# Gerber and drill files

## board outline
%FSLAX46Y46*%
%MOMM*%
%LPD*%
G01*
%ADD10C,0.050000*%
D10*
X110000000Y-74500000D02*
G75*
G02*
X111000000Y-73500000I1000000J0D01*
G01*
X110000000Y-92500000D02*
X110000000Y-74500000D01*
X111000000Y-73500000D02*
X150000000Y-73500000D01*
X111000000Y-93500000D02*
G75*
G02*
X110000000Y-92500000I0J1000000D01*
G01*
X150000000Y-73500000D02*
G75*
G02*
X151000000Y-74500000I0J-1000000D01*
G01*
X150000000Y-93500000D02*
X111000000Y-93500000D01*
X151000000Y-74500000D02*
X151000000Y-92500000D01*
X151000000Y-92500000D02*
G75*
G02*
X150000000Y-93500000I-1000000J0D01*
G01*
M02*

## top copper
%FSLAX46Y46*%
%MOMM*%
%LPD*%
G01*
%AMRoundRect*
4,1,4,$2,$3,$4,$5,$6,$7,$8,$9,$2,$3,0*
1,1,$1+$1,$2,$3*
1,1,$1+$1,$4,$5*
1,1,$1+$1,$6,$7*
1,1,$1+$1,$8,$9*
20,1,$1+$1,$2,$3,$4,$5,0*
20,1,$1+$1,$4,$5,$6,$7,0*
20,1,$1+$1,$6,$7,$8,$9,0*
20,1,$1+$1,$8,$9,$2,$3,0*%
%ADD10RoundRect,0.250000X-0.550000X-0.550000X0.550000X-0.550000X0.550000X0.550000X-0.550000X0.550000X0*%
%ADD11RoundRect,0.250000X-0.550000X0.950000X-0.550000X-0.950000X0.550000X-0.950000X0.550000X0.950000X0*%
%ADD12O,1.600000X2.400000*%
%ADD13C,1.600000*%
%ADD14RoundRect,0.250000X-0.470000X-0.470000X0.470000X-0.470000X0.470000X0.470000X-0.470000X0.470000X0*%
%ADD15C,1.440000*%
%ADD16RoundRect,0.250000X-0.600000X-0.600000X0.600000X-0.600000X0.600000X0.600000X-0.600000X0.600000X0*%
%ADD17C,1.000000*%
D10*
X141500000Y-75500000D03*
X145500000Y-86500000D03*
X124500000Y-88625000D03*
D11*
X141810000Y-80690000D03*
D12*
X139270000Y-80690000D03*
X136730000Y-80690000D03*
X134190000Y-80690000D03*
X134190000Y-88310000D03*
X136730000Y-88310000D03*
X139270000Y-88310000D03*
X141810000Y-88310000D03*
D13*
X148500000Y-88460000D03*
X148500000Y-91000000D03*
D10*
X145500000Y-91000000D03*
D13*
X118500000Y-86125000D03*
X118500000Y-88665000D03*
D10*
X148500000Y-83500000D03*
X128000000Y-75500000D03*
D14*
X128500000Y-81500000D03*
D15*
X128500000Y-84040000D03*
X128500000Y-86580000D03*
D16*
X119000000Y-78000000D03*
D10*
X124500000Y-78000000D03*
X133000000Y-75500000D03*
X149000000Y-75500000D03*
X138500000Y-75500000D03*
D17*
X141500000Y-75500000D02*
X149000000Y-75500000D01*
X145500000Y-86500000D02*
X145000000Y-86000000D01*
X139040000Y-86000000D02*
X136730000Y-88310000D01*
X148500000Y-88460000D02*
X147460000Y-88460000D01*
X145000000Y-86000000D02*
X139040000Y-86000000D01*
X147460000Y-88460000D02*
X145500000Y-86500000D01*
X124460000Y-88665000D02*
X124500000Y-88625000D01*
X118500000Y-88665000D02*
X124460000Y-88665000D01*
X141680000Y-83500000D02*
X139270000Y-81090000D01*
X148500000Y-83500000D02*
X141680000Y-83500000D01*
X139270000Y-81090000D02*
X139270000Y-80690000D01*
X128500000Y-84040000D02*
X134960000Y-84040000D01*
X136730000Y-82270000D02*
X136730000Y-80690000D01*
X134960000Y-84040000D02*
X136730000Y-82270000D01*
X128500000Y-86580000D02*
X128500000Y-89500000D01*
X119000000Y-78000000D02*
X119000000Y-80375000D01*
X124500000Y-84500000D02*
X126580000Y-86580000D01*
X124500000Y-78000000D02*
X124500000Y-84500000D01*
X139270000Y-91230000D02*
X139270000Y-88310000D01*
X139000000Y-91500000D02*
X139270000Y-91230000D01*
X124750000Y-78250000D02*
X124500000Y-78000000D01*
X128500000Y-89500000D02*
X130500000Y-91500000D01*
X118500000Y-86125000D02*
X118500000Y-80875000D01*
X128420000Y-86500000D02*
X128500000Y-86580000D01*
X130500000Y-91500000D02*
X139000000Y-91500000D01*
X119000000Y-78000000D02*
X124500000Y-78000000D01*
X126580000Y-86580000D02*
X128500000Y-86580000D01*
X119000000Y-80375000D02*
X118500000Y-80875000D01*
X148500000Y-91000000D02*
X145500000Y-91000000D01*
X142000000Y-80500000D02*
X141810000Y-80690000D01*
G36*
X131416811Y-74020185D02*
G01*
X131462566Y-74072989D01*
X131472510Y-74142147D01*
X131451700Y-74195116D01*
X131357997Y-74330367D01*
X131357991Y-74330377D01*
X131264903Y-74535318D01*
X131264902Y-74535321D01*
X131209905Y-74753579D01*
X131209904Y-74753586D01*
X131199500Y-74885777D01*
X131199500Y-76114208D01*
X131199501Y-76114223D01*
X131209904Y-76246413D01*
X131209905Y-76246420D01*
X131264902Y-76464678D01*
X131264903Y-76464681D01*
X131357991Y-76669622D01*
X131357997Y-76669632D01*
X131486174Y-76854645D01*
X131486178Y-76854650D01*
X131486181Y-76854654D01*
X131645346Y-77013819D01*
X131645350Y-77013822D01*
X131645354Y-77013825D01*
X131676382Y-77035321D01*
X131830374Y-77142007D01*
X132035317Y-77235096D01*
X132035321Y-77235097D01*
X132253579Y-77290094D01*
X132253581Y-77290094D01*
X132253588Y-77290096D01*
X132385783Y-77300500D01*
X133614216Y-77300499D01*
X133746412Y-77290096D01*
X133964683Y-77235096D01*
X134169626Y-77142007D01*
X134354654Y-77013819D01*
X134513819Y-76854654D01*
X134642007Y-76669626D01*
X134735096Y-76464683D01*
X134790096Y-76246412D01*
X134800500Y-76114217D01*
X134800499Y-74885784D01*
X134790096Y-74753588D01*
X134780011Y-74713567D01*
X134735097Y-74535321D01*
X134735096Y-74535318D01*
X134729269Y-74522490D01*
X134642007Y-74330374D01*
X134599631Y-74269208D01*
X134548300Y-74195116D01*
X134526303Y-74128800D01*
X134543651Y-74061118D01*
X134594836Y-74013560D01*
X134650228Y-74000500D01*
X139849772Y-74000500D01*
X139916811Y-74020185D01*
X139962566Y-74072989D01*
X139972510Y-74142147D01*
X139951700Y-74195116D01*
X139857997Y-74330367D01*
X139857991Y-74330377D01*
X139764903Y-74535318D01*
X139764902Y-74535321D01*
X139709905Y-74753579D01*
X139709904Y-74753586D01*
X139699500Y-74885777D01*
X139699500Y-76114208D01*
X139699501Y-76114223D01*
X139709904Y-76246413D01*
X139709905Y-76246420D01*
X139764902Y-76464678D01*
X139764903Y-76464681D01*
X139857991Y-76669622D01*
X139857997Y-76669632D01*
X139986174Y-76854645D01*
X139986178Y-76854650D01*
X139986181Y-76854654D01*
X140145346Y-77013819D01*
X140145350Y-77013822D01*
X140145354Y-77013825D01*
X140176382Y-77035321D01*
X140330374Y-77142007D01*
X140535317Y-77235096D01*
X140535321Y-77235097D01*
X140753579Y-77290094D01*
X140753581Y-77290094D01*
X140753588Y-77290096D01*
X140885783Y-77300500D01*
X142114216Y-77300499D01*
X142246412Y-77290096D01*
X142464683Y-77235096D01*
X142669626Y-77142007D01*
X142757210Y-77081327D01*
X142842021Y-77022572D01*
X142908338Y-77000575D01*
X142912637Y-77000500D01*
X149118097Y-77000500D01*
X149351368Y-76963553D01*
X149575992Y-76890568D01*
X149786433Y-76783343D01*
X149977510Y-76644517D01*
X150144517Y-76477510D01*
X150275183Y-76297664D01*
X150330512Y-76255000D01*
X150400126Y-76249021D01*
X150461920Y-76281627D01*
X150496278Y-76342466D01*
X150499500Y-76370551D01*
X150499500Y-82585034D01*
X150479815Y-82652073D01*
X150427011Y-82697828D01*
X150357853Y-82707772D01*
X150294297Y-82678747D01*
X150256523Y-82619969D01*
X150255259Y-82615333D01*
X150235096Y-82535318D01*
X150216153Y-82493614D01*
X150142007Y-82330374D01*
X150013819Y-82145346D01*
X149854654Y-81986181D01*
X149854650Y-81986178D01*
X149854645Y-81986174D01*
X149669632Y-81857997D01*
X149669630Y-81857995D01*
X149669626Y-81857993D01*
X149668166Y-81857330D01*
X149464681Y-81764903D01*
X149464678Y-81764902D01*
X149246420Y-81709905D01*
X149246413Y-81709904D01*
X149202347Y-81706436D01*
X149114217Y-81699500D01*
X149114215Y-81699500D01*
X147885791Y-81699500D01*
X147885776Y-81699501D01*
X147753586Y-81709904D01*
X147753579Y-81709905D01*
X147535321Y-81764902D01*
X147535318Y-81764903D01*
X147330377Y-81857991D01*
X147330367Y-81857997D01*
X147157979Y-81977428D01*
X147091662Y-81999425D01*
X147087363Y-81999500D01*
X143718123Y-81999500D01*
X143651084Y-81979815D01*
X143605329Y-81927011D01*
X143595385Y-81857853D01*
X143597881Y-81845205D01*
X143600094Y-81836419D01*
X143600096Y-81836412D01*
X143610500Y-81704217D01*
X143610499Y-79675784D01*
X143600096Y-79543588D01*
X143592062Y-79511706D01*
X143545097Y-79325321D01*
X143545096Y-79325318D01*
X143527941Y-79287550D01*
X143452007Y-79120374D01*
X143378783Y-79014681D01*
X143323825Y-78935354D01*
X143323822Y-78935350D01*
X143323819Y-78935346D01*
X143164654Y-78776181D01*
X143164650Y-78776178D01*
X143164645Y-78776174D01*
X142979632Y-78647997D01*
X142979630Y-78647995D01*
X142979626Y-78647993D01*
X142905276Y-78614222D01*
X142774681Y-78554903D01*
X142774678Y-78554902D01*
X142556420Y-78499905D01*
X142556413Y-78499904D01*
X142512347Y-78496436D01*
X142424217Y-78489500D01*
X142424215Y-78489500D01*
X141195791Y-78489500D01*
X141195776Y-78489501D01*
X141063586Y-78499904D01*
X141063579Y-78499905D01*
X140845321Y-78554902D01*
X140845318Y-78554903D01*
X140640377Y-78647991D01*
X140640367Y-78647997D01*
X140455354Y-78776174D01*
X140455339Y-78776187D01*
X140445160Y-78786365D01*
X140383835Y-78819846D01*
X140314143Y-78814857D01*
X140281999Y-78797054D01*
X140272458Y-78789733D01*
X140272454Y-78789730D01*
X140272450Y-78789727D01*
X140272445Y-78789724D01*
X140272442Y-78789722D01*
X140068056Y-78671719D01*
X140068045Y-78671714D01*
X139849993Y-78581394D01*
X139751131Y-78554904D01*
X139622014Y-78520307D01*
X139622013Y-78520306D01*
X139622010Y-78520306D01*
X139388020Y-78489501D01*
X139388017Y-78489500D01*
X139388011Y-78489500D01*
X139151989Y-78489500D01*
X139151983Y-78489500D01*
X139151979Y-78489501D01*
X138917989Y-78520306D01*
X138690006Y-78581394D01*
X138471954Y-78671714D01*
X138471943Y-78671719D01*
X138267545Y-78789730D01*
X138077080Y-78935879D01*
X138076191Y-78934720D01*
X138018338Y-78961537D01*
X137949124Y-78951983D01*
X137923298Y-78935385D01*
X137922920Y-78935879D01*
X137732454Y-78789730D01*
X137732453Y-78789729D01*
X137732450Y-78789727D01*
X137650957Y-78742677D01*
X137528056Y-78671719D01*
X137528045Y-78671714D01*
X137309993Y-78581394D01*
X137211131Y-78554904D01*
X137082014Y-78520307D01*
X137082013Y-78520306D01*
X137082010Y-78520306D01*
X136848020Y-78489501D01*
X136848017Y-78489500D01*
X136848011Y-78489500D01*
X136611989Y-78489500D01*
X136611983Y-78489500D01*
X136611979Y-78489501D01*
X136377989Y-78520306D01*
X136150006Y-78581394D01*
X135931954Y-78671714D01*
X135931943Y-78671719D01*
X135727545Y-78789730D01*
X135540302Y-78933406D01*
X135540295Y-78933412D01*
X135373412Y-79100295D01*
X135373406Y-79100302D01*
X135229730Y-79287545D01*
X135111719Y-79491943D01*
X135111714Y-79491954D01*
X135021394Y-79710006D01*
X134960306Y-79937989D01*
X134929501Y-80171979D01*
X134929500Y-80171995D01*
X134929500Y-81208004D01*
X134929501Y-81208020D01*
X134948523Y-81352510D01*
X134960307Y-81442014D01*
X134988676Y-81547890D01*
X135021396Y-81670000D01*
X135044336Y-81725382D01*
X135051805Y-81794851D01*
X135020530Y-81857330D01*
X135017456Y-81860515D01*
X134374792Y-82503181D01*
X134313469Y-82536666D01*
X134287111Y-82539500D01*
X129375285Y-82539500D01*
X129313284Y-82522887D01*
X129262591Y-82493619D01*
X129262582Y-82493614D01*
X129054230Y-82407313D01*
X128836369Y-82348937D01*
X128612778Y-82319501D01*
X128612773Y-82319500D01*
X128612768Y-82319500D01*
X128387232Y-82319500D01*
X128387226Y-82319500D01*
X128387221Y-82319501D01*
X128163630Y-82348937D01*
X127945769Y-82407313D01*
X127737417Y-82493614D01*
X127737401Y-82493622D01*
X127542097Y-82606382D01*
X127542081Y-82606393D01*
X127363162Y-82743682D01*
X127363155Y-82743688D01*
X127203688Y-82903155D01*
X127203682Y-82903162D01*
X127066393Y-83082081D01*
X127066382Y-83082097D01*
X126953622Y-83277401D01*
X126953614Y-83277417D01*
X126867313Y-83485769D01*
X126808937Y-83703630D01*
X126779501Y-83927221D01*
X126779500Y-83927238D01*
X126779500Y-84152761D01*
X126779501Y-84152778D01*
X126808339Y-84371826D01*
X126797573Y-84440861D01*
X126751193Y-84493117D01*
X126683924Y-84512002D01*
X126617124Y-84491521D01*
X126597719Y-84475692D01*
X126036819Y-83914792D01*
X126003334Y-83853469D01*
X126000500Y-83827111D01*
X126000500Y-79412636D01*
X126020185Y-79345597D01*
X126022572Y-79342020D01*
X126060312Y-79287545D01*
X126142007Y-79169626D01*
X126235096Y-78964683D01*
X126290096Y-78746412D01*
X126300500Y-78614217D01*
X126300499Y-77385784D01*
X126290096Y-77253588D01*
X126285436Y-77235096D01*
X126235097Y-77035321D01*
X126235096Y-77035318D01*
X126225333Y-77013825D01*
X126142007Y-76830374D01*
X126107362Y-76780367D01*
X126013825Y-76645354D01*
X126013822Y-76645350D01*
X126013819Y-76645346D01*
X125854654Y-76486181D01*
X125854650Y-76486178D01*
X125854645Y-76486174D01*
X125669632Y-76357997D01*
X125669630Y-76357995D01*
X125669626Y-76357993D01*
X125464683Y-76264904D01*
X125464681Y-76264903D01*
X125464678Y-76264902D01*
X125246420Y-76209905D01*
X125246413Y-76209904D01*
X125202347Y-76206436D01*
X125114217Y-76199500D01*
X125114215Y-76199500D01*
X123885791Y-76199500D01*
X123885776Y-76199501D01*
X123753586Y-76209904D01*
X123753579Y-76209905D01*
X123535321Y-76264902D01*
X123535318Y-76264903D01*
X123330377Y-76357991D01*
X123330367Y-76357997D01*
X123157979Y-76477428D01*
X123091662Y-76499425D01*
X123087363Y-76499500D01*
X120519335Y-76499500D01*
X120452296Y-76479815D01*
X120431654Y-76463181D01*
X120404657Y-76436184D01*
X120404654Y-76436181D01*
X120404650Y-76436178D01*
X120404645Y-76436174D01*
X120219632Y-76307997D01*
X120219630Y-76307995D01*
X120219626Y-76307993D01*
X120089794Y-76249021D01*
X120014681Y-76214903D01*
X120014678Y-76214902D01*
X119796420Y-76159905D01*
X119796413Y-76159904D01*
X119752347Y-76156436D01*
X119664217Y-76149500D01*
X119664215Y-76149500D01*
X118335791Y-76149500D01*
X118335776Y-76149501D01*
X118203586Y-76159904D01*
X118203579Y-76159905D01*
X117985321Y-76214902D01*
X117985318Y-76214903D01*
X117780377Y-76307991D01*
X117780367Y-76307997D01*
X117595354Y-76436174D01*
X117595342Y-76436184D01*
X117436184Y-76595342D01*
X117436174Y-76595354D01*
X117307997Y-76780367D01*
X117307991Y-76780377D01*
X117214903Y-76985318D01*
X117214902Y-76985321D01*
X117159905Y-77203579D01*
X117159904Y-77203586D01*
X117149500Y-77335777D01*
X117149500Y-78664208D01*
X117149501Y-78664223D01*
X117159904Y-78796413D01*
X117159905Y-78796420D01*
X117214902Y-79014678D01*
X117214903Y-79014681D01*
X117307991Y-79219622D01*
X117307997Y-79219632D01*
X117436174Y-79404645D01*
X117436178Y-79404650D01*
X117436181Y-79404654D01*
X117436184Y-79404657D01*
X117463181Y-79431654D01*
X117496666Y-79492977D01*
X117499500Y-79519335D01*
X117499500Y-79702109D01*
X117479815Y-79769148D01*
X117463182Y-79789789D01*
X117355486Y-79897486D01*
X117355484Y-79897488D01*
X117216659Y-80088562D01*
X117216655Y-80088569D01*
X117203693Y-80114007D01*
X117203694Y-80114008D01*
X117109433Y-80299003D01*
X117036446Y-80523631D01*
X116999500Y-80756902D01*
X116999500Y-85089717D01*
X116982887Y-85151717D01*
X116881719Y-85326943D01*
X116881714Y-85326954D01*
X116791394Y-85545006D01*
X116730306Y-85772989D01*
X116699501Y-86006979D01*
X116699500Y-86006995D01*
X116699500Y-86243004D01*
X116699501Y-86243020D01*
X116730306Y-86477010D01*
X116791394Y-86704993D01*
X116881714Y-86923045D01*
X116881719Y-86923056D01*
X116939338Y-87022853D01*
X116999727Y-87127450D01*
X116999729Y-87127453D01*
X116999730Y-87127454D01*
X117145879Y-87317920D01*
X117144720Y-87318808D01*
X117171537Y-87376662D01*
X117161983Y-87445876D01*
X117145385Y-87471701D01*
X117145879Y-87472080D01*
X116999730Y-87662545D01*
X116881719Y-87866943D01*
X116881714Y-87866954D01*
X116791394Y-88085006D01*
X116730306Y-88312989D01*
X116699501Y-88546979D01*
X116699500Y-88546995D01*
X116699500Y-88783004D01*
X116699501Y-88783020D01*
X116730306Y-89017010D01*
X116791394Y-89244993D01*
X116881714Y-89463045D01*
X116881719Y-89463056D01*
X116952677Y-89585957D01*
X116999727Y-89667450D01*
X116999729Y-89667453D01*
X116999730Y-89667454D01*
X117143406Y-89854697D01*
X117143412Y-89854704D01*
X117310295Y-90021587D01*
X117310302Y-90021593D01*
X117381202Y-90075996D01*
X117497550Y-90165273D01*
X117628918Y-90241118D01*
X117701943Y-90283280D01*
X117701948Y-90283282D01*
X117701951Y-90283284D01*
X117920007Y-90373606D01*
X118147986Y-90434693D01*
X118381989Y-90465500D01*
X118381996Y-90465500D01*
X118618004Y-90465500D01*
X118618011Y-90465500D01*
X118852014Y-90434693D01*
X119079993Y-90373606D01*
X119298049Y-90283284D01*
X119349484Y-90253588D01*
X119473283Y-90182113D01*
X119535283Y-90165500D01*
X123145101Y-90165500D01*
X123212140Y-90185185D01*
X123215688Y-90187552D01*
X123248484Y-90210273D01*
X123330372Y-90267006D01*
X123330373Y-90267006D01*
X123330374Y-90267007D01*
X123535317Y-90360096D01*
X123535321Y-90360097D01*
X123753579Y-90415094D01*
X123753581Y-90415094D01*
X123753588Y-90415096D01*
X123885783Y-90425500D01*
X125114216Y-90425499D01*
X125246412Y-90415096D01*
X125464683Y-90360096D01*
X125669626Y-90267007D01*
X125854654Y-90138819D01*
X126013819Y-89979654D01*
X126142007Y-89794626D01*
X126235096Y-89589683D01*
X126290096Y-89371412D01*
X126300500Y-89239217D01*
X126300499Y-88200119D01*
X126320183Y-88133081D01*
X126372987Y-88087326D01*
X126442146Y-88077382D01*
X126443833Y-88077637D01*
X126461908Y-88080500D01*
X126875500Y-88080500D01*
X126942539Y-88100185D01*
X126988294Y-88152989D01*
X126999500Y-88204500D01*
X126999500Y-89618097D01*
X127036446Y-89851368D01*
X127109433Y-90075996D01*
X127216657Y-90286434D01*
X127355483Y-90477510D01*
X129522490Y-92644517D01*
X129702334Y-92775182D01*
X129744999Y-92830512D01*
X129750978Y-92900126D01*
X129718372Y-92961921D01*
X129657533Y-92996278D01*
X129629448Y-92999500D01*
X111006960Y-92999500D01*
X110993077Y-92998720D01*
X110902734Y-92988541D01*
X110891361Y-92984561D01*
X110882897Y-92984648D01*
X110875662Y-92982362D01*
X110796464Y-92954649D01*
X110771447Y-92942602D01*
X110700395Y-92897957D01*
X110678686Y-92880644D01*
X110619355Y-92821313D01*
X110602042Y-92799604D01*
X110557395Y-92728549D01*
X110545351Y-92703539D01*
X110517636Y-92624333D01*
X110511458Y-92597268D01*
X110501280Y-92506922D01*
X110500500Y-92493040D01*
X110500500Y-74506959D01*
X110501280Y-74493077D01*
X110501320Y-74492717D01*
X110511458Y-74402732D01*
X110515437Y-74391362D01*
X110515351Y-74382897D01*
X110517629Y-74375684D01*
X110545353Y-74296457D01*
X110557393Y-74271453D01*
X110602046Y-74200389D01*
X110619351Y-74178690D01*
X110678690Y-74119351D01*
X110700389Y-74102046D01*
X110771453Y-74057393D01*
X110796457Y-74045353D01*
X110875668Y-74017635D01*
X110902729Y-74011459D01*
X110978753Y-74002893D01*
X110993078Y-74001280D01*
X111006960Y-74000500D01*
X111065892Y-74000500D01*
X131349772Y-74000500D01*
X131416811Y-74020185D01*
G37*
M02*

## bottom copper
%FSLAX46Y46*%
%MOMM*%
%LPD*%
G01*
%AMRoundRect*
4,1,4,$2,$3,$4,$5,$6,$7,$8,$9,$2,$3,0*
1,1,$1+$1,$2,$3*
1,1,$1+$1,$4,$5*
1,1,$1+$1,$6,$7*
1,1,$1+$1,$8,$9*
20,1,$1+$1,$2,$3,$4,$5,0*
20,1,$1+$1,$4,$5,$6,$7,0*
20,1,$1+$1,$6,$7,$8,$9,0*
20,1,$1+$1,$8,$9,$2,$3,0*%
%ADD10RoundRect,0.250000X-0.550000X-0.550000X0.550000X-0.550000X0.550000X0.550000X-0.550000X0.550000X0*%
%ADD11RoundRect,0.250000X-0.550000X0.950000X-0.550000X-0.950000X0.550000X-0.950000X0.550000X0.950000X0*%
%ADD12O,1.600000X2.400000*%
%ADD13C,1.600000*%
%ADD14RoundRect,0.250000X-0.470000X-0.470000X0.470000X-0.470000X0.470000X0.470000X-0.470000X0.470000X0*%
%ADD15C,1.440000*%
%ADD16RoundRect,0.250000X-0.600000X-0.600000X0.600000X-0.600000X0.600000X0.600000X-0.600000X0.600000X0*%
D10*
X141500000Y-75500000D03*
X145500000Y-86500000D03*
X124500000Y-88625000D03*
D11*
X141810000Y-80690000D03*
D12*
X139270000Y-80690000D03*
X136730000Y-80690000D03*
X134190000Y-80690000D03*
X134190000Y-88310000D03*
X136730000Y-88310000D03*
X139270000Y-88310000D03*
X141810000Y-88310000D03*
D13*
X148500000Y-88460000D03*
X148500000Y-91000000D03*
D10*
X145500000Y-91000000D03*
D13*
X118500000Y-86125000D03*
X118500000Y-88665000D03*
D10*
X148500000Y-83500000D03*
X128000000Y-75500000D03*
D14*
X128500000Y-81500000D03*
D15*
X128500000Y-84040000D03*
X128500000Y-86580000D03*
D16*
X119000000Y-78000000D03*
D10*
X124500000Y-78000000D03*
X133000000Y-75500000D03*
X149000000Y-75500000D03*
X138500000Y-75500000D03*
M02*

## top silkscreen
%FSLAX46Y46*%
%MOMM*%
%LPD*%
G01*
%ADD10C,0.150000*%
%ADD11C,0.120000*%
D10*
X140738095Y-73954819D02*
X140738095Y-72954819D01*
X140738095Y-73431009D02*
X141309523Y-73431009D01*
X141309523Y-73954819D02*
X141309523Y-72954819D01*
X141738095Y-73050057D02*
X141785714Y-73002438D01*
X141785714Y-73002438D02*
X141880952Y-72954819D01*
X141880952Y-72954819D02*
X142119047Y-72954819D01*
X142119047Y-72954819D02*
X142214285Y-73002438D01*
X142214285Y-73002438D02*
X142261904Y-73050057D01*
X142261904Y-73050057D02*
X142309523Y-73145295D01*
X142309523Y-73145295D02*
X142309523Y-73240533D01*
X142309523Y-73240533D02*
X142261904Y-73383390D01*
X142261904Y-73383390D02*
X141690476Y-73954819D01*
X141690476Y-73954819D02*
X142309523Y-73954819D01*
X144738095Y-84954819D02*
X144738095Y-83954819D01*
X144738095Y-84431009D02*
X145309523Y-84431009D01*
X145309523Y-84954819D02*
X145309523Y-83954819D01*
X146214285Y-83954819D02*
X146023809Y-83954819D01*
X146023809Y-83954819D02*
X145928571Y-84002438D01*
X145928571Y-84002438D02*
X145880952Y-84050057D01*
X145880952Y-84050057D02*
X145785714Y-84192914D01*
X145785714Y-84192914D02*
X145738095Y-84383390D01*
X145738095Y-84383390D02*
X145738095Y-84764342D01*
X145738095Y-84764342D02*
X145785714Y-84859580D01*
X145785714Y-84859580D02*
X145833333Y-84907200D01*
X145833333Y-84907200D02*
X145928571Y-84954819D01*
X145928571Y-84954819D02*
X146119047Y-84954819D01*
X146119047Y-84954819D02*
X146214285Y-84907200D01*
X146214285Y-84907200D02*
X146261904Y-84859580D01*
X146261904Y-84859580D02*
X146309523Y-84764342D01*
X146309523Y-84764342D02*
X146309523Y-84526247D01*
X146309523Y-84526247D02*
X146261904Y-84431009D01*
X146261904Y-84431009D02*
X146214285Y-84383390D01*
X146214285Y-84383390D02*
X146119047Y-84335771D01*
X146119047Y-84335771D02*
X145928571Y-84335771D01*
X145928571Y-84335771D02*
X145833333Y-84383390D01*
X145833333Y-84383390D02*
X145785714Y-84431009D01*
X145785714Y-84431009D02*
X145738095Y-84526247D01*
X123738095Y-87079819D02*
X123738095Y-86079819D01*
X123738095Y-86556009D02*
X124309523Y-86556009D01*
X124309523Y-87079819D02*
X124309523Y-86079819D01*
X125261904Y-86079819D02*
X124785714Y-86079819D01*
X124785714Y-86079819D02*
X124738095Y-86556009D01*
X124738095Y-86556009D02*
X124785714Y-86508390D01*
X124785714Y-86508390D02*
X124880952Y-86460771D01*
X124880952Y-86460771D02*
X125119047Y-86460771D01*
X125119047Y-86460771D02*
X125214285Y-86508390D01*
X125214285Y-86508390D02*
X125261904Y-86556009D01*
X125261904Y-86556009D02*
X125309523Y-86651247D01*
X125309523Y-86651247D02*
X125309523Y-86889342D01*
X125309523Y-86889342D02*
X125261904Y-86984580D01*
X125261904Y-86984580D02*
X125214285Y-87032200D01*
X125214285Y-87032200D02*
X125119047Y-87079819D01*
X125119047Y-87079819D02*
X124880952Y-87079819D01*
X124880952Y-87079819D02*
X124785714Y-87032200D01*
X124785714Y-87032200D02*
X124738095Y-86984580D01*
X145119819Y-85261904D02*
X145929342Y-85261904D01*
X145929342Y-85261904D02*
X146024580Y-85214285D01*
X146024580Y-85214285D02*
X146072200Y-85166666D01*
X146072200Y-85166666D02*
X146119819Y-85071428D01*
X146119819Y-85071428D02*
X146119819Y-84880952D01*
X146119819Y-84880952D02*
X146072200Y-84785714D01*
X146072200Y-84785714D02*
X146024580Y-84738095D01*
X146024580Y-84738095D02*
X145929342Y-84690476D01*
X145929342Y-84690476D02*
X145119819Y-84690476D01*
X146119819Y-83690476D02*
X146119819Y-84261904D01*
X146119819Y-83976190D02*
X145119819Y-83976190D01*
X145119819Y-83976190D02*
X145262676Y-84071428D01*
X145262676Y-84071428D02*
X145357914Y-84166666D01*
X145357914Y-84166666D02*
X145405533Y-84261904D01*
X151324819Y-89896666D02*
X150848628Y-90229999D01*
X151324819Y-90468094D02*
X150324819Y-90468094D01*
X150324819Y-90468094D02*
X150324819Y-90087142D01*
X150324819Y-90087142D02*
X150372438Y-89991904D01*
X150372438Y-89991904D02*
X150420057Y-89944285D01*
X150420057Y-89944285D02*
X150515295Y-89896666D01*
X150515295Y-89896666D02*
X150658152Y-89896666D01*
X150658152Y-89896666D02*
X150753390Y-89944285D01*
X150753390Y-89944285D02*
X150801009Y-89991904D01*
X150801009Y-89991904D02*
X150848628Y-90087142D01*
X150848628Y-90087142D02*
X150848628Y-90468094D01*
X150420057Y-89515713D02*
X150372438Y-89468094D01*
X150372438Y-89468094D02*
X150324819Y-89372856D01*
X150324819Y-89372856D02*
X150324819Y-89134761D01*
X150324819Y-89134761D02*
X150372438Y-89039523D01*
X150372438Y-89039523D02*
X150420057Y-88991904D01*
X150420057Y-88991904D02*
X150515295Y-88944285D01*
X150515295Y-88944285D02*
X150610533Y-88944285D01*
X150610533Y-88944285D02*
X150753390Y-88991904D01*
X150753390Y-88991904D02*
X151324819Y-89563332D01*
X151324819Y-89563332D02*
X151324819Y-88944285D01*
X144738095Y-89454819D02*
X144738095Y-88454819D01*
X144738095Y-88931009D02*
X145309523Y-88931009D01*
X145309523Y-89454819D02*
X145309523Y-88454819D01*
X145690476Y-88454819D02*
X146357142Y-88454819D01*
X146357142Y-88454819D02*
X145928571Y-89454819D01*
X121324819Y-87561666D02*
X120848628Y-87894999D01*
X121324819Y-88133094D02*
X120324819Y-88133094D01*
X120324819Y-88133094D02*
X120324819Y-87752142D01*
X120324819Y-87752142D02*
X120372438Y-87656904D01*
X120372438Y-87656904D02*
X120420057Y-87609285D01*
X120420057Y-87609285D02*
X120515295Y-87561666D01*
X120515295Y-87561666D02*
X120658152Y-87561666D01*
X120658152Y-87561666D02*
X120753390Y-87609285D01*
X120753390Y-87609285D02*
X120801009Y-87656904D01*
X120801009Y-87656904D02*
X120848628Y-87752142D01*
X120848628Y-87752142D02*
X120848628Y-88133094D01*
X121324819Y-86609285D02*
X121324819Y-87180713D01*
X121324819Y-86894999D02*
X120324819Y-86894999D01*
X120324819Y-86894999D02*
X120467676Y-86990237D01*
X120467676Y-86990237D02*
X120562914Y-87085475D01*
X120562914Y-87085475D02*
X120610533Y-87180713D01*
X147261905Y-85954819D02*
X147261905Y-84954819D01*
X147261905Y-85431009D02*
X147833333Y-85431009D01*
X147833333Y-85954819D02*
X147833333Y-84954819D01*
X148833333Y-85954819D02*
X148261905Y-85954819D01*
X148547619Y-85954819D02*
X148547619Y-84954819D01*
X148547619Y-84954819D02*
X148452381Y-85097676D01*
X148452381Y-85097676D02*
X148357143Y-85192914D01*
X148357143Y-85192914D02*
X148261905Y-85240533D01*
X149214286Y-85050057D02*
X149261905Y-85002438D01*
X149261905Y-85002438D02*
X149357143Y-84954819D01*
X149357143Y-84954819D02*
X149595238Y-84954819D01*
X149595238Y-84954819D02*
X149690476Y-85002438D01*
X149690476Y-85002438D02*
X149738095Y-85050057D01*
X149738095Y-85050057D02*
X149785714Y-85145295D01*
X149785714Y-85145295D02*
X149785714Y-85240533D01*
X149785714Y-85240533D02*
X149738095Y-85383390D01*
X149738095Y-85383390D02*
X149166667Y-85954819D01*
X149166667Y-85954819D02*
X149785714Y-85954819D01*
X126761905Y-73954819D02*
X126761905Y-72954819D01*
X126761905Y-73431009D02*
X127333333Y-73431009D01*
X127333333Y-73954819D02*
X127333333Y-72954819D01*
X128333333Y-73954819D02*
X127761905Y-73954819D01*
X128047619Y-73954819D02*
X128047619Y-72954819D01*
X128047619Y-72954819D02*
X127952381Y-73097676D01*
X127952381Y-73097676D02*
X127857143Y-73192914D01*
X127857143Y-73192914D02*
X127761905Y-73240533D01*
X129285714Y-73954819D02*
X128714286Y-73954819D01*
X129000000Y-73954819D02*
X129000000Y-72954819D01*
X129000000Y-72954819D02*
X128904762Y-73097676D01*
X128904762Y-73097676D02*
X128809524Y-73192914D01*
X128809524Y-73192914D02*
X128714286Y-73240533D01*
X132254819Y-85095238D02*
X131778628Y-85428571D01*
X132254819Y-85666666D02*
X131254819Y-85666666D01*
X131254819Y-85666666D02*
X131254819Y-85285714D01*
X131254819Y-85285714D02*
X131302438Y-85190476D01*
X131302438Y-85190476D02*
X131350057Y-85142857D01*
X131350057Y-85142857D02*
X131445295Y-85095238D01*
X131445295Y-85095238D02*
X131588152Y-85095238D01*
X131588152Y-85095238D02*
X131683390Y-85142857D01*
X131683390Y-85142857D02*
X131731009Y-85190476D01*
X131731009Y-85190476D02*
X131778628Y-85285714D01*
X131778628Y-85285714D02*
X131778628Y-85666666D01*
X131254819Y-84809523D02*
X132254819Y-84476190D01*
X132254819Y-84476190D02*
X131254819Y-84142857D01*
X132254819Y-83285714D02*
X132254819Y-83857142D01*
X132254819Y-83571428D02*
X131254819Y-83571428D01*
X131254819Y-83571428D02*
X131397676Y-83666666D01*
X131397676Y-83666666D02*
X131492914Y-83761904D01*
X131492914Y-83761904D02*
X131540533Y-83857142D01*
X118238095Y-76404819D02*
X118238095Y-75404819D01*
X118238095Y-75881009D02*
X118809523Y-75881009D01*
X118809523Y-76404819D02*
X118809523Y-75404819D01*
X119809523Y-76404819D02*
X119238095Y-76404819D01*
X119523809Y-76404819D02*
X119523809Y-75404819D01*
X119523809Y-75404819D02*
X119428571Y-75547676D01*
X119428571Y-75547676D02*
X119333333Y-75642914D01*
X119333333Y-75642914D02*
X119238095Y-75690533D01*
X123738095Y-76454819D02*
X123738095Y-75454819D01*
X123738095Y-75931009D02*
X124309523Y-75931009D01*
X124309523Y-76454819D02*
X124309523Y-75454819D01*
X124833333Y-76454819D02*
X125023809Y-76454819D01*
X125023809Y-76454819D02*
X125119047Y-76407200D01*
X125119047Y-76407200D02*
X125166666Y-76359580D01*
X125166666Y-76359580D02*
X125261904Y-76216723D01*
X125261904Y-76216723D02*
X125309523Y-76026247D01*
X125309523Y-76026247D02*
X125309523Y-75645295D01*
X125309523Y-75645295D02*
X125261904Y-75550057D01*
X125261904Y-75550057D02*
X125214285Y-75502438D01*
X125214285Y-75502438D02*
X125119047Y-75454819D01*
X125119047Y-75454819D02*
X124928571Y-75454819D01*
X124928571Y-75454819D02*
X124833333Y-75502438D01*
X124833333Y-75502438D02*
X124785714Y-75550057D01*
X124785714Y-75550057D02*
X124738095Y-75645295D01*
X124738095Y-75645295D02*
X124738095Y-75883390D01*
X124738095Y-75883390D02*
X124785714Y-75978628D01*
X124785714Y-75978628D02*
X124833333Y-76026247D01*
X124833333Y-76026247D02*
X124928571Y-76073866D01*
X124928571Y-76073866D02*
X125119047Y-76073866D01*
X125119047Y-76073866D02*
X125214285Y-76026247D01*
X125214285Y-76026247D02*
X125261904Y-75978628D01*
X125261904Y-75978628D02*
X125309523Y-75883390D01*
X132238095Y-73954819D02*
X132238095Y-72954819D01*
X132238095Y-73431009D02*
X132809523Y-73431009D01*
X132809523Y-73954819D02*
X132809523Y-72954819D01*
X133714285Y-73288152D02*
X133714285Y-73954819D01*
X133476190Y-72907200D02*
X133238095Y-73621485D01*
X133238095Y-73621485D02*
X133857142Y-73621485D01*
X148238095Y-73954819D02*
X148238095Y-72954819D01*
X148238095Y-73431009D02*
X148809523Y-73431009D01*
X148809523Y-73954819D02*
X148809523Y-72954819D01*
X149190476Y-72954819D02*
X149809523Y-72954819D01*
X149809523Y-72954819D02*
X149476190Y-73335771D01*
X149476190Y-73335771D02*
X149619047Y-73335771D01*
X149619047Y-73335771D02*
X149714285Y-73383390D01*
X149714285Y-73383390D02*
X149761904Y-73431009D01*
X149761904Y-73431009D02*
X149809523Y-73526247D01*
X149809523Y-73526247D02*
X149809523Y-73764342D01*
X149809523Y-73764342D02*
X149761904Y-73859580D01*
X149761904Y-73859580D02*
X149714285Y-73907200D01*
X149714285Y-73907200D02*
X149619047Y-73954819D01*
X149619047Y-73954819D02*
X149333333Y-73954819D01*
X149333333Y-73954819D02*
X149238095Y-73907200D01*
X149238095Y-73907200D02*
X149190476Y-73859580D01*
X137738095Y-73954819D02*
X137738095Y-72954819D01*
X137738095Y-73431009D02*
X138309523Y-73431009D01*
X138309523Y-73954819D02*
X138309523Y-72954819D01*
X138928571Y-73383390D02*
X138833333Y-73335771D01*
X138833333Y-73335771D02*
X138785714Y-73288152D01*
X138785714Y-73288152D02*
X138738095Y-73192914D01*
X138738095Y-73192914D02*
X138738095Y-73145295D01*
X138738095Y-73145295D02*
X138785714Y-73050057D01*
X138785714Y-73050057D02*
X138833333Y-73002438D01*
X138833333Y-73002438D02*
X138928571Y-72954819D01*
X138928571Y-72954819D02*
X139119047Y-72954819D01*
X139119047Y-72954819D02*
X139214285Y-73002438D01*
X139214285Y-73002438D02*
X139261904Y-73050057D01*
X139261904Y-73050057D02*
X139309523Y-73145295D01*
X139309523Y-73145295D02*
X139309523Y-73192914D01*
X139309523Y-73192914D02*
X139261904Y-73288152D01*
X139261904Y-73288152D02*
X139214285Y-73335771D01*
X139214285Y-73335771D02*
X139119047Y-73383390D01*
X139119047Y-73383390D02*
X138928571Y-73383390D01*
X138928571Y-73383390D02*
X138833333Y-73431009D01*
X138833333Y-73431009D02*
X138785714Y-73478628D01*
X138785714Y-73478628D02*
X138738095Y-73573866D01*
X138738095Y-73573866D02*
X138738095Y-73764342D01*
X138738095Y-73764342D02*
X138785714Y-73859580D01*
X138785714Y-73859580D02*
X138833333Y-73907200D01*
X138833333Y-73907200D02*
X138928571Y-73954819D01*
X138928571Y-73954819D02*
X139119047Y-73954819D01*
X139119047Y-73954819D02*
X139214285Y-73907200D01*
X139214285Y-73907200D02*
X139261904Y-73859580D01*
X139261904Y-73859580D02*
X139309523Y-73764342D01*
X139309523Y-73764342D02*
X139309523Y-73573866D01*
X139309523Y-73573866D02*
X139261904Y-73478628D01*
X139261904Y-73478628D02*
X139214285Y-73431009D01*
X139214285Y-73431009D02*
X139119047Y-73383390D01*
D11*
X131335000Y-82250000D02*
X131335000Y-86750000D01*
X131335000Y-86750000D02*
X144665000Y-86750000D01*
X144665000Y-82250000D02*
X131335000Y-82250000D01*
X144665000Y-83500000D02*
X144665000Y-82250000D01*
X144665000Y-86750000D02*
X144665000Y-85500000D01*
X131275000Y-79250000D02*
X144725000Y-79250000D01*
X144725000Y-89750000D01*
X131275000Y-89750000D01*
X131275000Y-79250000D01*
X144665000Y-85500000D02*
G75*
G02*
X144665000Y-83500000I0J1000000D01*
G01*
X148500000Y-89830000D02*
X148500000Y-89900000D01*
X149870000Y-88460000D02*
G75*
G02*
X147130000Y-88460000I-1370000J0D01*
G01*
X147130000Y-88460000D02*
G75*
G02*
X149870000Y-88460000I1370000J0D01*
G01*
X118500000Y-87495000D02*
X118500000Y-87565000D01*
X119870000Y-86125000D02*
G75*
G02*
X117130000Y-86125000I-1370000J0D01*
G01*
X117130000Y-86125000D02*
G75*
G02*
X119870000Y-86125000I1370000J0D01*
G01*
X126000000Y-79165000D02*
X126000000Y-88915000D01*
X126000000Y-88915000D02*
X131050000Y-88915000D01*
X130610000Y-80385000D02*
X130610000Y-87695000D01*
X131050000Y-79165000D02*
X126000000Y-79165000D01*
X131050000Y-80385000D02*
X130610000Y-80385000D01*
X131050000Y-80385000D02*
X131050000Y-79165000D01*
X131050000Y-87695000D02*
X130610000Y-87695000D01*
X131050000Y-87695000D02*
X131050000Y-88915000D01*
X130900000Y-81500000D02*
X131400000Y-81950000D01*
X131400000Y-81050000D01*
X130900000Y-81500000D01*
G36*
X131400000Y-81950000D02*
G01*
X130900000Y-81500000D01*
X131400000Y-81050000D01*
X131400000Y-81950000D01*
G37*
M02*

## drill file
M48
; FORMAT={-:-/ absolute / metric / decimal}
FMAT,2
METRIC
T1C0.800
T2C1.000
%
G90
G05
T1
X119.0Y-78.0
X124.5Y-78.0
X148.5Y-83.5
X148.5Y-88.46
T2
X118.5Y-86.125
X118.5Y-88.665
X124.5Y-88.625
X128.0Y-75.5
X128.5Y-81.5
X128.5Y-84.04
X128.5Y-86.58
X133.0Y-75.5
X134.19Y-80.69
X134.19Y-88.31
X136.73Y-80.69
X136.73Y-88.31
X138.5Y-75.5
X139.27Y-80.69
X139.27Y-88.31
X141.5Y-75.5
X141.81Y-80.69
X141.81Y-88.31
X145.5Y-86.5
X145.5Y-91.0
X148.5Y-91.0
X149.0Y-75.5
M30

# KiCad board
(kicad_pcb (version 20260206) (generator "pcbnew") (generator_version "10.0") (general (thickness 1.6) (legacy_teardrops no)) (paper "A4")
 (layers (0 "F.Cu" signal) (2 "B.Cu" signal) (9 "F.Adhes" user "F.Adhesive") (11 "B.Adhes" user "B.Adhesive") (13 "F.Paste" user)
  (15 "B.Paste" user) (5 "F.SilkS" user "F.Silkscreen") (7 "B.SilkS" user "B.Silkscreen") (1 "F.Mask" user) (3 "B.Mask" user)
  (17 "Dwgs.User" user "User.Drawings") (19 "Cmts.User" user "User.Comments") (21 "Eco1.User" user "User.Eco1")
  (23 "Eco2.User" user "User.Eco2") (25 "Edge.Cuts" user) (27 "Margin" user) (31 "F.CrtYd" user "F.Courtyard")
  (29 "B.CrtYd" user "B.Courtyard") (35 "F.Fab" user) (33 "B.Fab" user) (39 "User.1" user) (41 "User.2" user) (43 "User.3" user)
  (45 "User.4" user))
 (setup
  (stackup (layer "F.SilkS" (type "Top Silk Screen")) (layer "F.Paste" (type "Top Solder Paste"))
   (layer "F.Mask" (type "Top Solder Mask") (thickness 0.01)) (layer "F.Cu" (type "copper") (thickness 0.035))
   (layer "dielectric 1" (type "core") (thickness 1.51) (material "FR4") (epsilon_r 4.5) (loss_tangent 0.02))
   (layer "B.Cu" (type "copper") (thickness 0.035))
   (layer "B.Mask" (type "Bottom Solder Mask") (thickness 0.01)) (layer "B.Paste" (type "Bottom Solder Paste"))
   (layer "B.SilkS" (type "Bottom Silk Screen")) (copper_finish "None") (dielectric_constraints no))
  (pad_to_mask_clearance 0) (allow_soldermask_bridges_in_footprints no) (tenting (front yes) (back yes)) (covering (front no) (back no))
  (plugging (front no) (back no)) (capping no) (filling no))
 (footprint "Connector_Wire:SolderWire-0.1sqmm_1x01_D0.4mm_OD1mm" (layer "F.Cu") (at 141.5 75.5)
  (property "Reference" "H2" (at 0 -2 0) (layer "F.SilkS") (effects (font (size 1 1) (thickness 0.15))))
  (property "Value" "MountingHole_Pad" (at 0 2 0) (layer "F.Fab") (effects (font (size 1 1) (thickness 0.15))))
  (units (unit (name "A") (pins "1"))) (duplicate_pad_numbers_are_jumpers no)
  (pad "1" thru_hole roundrect (at 0 0) (size 1.6 1.6) (drill 1) (layers "*.Cu" "*.Mask") (remove_unused_layers no)
   (roundrect_rratio 0.15625) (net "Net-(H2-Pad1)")))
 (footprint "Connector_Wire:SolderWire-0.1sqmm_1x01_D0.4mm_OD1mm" (layer "F.Cu") (at 145.5 86.5)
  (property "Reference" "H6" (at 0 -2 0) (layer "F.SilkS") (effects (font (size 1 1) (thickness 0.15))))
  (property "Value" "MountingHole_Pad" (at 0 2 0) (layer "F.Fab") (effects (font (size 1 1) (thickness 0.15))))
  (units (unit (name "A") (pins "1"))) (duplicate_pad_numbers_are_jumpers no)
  (pad "1" thru_hole roundrect (at 0 0) (size 1.6 1.6) (drill 1) (layers "*.Cu" "*.Mask") (remove_unused_layers no)
   (roundrect_rratio 0.15625) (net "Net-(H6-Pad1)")))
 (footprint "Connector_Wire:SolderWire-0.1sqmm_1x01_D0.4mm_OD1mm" (layer "F.Cu") (at 124.5 88.625)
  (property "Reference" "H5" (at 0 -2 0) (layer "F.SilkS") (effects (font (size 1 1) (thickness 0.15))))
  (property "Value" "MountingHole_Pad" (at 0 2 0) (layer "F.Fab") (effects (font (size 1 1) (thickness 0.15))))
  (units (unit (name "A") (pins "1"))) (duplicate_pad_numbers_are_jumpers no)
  (pad "1" thru_hole roundrect (at 0 0) (size 1.6 1.6) (drill 1) (layers "*.Cu" "*.Mask") (remove_unused_layers no)
   (roundrect_rratio 0.15625) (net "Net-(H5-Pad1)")))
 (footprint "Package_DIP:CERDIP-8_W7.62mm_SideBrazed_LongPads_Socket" (layer "F.Cu") (at 141.81 80.69 -90)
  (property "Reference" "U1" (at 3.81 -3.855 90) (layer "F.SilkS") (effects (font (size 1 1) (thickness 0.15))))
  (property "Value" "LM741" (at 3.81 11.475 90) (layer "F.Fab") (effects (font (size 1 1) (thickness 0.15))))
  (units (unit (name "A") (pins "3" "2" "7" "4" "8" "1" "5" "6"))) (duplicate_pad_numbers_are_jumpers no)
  (fp_line (start 1.56 10.475) (end 6.06 10.475) (stroke (width 0.12) (type solid)) (layer "F.SilkS"))
  (fp_line (start 6.06 10.475) (end 6.06 -2.855) (stroke (width 0.12) (type solid)) (layer "F.SilkS"))
  (fp_line (start 1.56 -2.855) (end 1.56 10.475) (stroke (width 0.12) (type solid)) (layer "F.SilkS"))
  (fp_line (start 2.81 -2.855) (end 1.56 -2.855) (stroke (width 0.12) (type solid)) (layer "F.SilkS"))
  (fp_line (start 6.06 -2.855) (end 4.81 -2.855) (stroke (width 0.12) (type solid)) (layer "F.SilkS"))
  (fp_rect (start -1.44 -2.915) (end 9.06 10.535) (stroke (width 0.12) (type solid)) (fill no) (layer "F.SilkS"))
  (fp_arc (start 4.81 -2.855) (mid 3.81 -1.855) (end 2.81 -2.855) (stroke (width 0.12) (type solid)) (layer "F.SilkS"))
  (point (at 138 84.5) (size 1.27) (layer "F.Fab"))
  (pad "1" thru_hole roundrect (at 0 0 270) (size 2.4 1.6) (drill 1) (layers "*.Cu" "*.Mask") (remove_unused_layers no)
   (roundrect_rratio 0.15625) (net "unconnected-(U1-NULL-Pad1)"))
  (pad "2" thru_hole oval (at 0 2.54 270) (size 2.4 1.6) (drill 1) (layers "*.Cu" "*.Mask") (remove_unused_layers no) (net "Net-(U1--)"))
  (pad "3" thru_hole oval (at 0 5.08 270) (size 2.4 1.6) (drill 1) (layers "*.Cu" "*.Mask") (remove_unused_layers no) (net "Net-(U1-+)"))
  (pad "4" thru_hole oval (at 0 7.62 270) (size 2.4 1.6) (drill 1) (layers "*.Cu" "*.Mask") (remove_unused_layers no) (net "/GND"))
  (pad "5" thru_hole oval (at 7.62 7.62 270) (size 2.4 1.6) (drill 1) (layers "*.Cu" "*.Mask") (remove_unused_layers no)
   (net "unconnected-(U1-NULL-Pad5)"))
  (pad "6" thru_hole oval (at 7.62 5.08 270) (size 2.4 1.6) (drill 1) (layers "*.Cu" "*.Mask") (remove_unused_layers no)
   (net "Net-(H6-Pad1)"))
  (pad "7" thru_hole oval (at 7.62 2.54 270) (size 2.4 1.6) (drill 1) (layers "*.Cu" "*.Mask") (remove_unused_layers no) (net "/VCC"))
  (pad "8" thru_hole oval (at 7.62 0 270) (size 2.4 1.6) (drill 1) (layers "*.Cu" "*.Mask") (remove_unused_layers no)
   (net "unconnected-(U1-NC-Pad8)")))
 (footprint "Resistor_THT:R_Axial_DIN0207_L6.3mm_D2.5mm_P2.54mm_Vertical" (layer "F.Cu") (at 148.5 88.46 -90)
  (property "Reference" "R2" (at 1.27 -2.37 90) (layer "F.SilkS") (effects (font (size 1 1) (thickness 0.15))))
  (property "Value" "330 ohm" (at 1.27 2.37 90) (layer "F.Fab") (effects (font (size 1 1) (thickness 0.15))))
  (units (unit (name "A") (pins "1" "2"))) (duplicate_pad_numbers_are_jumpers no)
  (fp_line (start 1.37 0) (end 1.44 0) (stroke (width 0.12) (type solid)) (layer "F.SilkS"))
  (fp_circle (center 0 0) (end 1.37 0) (stroke (width 0.12) (type solid)) (fill no) (layer "F.SilkS"))
  (pad "1" thru_hole circle (at 0 0 270) (size 1.6 1.6) (drill 0.8) (layers "*.Cu" "*.Mask") (remove_unused_layers no) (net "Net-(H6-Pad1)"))
  (pad "2" thru_hole circle (at 2.54 0 270) (size 1.6 1.6) (drill 1) (layers "*.Cu" "*.Mask") (remove_unused_layers no)
   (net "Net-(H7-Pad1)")))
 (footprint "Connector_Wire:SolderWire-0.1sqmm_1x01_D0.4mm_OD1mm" (layer "F.Cu") (at 145.5 91)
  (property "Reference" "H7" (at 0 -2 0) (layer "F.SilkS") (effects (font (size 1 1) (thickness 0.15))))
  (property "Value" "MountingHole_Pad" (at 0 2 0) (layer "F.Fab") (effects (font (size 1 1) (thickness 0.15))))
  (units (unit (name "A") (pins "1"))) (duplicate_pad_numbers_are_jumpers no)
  (pad "1" thru_hole roundrect (at 0 0) (size 1.6 1.6) (drill 1) (layers "*.Cu" "*.Mask") (remove_unused_layers no)
   (roundrect_rratio 0.15625) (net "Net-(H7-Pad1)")))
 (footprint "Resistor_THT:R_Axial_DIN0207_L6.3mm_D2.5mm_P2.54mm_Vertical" (layer "F.Cu") (at 118.5 86.125 -90)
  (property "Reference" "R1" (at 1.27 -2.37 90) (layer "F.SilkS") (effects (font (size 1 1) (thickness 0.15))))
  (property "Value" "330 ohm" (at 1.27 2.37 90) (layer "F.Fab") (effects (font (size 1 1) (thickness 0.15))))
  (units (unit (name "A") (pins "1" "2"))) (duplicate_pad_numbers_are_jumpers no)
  (fp_line (start 1.37 0) (end 1.44 0) (stroke (width 0.12) (type solid)) (layer "F.SilkS"))
  (fp_circle (center 0 0) (end 1.37 0) (stroke (width 0.12) (type solid)) (fill no) (layer "F.SilkS"))
  (pad "1" thru_hole circle (at 0 0 270) (size 1.6 1.6) (drill 1) (layers "*.Cu" "*.Mask") (remove_unused_layers no) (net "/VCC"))
  (pad "2" thru_hole circle (at 2.54 0 270) (size 1.6 1.6) (drill 1) (layers "*.Cu" "*.Mask") (remove_unused_layers no)
   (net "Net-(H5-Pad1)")))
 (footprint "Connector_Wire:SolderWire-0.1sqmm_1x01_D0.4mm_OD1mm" (layer "F.Cu") (at 148.5 83.5)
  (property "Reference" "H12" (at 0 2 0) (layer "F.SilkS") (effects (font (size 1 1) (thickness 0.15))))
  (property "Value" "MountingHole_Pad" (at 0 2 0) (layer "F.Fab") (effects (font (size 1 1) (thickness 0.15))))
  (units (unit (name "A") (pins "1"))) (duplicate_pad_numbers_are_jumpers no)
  (pad "1" thru_hole roundrect (at 0 0) (size 1.6 1.6) (drill 0.8) (layers "*.Cu" "*.Mask") (remove_unused_layers no)
   (roundrect_rratio 0.15625) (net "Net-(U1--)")))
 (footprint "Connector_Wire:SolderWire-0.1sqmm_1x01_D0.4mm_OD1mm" (layer "F.Cu") (at 128 75.5)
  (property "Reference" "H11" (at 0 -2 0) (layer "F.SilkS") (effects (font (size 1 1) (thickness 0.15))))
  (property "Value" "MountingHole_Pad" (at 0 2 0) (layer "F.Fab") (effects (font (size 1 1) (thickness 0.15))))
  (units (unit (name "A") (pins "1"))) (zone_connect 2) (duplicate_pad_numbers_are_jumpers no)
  (pad "1" thru_hole roundrect (at 0 0) (size 1.6 1.6) (drill 1) (layers "*.Cu" "*.Mask") (remove_unused_layers no)
   (roundrect_rratio 0.15625) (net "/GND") (zone_connect 2)))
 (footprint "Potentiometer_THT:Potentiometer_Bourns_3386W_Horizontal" (layer "F.Cu") (at 128.5 81.5 -90)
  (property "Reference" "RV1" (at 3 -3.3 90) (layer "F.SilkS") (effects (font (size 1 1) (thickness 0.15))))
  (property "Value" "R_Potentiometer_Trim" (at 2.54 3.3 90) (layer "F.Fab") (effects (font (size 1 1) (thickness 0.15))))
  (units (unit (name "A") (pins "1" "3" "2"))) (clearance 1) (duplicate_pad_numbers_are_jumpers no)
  (fp_line (start -2.335 2.5) (end 7.415 2.5) (stroke (width 0.12) (type default)) (layer "F.SilkS"))
  (fp_line (start 7.415 2.5) (end 7.415 -2.55) (stroke (width 0.12) (type default)) (layer "F.SilkS"))
  (fp_line (start -1.115 -2.11) (end 6.195 -2.11) (stroke (width 0.12) (type default)) (layer "F.SilkS"))
  (fp_line (start -2.335 -2.55) (end -2.335 2.5) (stroke (width 0.12) (type default)) (layer "F.SilkS"))
  (fp_line (start -1.115 -2.55) (end -1.115 -2.11) (stroke (width 0.12) (type default)) (layer "F.SilkS"))
  (fp_line (start -1.115 -2.55) (end -2.335 -2.55) (stroke (width 0.12) (type default)) (layer "F.SilkS"))
  (fp_line (start 6.195 -2.55) (end 6.195 -2.11) (stroke (width 0.12) (type default)) (layer "F.SilkS"))
  (fp_line (start 6.195 -2.55) (end 7.415 -2.55) (stroke (width 0.12) (type default)) (layer "F.SilkS"))
  (fp_poly (pts (xy 0 -2.4) (xy 0.45 -2.9) (xy -0.45 -2.9)) (stroke (width 0.12) (type solid)) (fill yes) (layer "F.SilkS"))
  (pad "1" thru_hole roundrect (at 0 0) (size 1.44 1.44) (drill 1) (layers "*.Cu" "*.Mask") (remove_unused_layers no)
   (roundrect_rratio 0.1736111111) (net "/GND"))
  (pad "2" thru_hole circle (at 2.54 0) (size 1.44 1.44) (drill 1) (layers "*.Cu" "*.Mask") (remove_unused_layers no) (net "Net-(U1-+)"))
  (pad "3" thru_hole circle (at 5.08 0) (size 1.44 1.44) (drill 1) (layers "*.Cu" "*.Mask") (remove_unused_layers no) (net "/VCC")))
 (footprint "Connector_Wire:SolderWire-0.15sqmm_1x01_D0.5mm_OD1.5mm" (layer "F.Cu") (at 119 78)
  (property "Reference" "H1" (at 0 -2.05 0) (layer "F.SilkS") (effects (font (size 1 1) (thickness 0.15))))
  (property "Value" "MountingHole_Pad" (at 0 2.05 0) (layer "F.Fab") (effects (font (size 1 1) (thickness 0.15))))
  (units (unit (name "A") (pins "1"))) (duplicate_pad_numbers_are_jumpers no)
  (pad "1" thru_hole roundrect (at 0 0) (size 1.7 1.7) (drill 0.8) (layers "*.Cu" "*.Mask") (remove_unused_layers no)
   (roundrect_rratio 0.147059) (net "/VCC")))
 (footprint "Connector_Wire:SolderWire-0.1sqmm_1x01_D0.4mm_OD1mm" (layer "F.Cu") (at 124.5 78)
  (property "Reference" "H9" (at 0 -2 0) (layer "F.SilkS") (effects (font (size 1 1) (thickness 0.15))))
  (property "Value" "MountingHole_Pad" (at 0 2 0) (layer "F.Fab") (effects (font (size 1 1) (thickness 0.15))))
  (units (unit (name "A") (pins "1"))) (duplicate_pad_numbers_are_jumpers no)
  (pad "1" thru_hole roundrect (at 0 0) (size 1.6 1.6) (drill 0.8) (layers "*.Cu" "*.Mask") (remove_unused_layers no)
   (roundrect_rratio 0.15625) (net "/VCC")))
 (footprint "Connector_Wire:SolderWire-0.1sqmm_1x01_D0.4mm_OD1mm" (layer "F.Cu") (at 133 75.5)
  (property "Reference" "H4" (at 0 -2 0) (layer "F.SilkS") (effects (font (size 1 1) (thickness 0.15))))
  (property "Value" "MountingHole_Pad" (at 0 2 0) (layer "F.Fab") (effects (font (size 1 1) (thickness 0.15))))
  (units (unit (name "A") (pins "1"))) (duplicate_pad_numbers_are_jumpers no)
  (pad "1" thru_hole roundrect (at 0 0) (size 1.6 1.6) (drill 1) (layers "*.Cu" "*.Mask") (remove_unused_layers no)
   (roundrect_rratio 0.15625) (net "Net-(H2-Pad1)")))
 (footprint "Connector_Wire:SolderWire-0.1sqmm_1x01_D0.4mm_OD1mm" (layer "F.Cu") (at 149 75.5)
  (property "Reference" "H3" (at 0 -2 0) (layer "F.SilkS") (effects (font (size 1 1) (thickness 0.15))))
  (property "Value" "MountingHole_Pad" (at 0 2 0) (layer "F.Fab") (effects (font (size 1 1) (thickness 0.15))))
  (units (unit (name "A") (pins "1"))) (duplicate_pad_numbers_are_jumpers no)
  (pad "1" thru_hole roundrect (at 0 0) (size 1.6 1.6) (drill 1) (layers "*.Cu" "*.Mask") (remove_unused_layers no)
   (roundrect_rratio 0.15625) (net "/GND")))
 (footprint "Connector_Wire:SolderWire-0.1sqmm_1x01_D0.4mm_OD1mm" (layer "F.Cu") (at 138.5 75.5)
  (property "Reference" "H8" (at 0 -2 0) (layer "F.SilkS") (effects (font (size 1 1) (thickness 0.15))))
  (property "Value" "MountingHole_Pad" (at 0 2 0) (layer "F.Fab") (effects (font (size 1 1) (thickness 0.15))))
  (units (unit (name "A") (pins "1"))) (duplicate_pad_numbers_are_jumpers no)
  (pad "1" thru_hole roundrect (at 0 0) (size 1.6 1.6) (drill 1) (layers "*.Cu" "*.Mask") (remove_unused_layers no)
   (roundrect_rratio 0.15625) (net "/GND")))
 (gr_arc (start 110 74.5) (mid 110.292893 73.792893) (end 111 73.5) (stroke (width 0.05) (type default)) (layer "Edge.Cuts"))
 (gr_line (start 110 92.5) (end 110 74.5) (stroke (width 0.05) (type default)) (layer "Edge.Cuts"))
 (gr_line (start 111 73.5) (end 150 73.5) (stroke (width 0.05) (type default)) (layer "Edge.Cuts"))
 (gr_arc (start 111 93.5) (mid 110.292893 93.207107) (end 110 92.5) (stroke (width 0.05) (type default)) (layer "Edge.Cuts"))
 (gr_arc (start 150 73.5) (mid 150.707107 73.792893) (end 151 74.5) (stroke (width 0.05) (type default)) (layer "Edge.Cuts"))
 (gr_line (start 150 93.5) (end 111 93.5) (stroke (width 0.05) (type default)) (layer "Edge.Cuts"))
 (gr_line (start 151 74.5) (end 151 92.5) (stroke (width 0.05) (type default)) (layer "Edge.Cuts"))
 (gr_arc (start 151 92.5) (mid 150.707107 93.207107) (end 150 93.5) (stroke (width 0.05) (type default)) (layer "Edge.Cuts"))
 (segment (start 141.5 75.5) (end 149 75.5) (width 1) (layer "F.Cu") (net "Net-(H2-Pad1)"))
 (segment (start 145.5 86.5) (end 145 86) (width 1) (layer "F.Cu") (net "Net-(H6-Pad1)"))
 (segment (start 139.04 86) (end 136.73 88.31) (width 1) (layer "F.Cu") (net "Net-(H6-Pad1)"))
 (segment (start 148.5 88.46) (end 147.46 88.46) (width 1) (layer "F.Cu") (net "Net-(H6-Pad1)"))
 (segment (start 145 86) (end 139.04 86) (width 1) (layer "F.Cu") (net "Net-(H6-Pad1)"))
 (segment (start 147.46 88.46) (end 145.5 86.5) (width 1) (layer "F.Cu") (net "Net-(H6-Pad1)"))
 (segment (start 124.46 88.665) (end 124.5 88.625) (width 1) (layer "F.Cu") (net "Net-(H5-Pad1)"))
 (segment (start 118.5 88.665) (end 124.46 88.665) (width 1) (layer "F.Cu") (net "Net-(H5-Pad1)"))
 (segment (start 141.68 83.5) (end 139.27 81.09) (width 1) (layer "F.Cu") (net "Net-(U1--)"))
 (segment (start 148.5 83.5) (end 141.68 83.5) (width 1) (layer "F.Cu") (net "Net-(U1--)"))
 (segment (start 139.27 81.09) (end 139.27 80.69) (width 1) (layer "F.Cu") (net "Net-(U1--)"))
 (segment (start 128.5 84.04) (end 134.96 84.04) (width 1) (layer "F.Cu") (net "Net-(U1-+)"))
 (segment (start 136.73 82.27) (end 136.73 80.69) (width 1) (layer "F.Cu") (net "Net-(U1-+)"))
 (segment (start 134.96 84.04) (end 136.73 82.27) (width 1) (layer "F.Cu") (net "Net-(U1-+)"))
 (segment (start 128.5 86.58) (end 128.5 89.5) (width 1) (layer "F.Cu") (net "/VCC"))
 (segment (start 119 78) (end 119 80.375) (width 1) (layer "F.Cu") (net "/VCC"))
 (segment (start 124.5 84.5) (end 126.58 86.58) (width 1) (layer "F.Cu") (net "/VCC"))
 (segment (start 124.5 78) (end 124.5 84.5) (width 1) (layer "F.Cu") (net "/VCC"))
 (segment (start 139.27 91.23) (end 139.27 88.31) (width 1) (layer "F.Cu") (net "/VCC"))
 (segment (start 139 91.5) (end 139.27 91.23) (width 1) (layer "F.Cu") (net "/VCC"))
 (segment (start 124.75 78.25) (end 124.5 78) (width 1) (layer "F.Cu") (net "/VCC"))
 (segment (start 128.5 89.5) (end 130.5 91.5) (width 1) (layer "F.Cu") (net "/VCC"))
 (segment (start 118.5 86.125) (end 118.5 80.875) (width 1) (layer "F.Cu") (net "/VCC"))
 (segment (start 128.42 86.5) (end 128.5 86.58) (width 1) (layer "F.Cu") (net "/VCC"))
 (segment (start 130.5 91.5) (end 139 91.5) (width 1) (layer "F.Cu") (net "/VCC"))
 (segment (start 119 78) (end 124.5 78) (width 1) (layer "F.Cu") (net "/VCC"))
 (segment (start 126.58 86.58) (end 128.5 86.58) (width 1) (layer "F.Cu") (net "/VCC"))
 (segment (start 119 80.375) (end 118.5 80.875) (width 1) (layer "F.Cu") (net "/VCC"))
 (segment (start 148.5 91) (end 145.5 91) (width 1) (layer "F.Cu") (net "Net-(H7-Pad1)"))
 (segment (start 142 80.5) (end 141.81 80.69) (width 1) (layer "F.Cu") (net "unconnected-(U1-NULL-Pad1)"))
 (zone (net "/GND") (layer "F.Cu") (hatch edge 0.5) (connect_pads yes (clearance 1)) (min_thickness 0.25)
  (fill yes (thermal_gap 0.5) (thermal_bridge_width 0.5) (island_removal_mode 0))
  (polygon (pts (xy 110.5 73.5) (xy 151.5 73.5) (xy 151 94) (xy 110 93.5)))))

